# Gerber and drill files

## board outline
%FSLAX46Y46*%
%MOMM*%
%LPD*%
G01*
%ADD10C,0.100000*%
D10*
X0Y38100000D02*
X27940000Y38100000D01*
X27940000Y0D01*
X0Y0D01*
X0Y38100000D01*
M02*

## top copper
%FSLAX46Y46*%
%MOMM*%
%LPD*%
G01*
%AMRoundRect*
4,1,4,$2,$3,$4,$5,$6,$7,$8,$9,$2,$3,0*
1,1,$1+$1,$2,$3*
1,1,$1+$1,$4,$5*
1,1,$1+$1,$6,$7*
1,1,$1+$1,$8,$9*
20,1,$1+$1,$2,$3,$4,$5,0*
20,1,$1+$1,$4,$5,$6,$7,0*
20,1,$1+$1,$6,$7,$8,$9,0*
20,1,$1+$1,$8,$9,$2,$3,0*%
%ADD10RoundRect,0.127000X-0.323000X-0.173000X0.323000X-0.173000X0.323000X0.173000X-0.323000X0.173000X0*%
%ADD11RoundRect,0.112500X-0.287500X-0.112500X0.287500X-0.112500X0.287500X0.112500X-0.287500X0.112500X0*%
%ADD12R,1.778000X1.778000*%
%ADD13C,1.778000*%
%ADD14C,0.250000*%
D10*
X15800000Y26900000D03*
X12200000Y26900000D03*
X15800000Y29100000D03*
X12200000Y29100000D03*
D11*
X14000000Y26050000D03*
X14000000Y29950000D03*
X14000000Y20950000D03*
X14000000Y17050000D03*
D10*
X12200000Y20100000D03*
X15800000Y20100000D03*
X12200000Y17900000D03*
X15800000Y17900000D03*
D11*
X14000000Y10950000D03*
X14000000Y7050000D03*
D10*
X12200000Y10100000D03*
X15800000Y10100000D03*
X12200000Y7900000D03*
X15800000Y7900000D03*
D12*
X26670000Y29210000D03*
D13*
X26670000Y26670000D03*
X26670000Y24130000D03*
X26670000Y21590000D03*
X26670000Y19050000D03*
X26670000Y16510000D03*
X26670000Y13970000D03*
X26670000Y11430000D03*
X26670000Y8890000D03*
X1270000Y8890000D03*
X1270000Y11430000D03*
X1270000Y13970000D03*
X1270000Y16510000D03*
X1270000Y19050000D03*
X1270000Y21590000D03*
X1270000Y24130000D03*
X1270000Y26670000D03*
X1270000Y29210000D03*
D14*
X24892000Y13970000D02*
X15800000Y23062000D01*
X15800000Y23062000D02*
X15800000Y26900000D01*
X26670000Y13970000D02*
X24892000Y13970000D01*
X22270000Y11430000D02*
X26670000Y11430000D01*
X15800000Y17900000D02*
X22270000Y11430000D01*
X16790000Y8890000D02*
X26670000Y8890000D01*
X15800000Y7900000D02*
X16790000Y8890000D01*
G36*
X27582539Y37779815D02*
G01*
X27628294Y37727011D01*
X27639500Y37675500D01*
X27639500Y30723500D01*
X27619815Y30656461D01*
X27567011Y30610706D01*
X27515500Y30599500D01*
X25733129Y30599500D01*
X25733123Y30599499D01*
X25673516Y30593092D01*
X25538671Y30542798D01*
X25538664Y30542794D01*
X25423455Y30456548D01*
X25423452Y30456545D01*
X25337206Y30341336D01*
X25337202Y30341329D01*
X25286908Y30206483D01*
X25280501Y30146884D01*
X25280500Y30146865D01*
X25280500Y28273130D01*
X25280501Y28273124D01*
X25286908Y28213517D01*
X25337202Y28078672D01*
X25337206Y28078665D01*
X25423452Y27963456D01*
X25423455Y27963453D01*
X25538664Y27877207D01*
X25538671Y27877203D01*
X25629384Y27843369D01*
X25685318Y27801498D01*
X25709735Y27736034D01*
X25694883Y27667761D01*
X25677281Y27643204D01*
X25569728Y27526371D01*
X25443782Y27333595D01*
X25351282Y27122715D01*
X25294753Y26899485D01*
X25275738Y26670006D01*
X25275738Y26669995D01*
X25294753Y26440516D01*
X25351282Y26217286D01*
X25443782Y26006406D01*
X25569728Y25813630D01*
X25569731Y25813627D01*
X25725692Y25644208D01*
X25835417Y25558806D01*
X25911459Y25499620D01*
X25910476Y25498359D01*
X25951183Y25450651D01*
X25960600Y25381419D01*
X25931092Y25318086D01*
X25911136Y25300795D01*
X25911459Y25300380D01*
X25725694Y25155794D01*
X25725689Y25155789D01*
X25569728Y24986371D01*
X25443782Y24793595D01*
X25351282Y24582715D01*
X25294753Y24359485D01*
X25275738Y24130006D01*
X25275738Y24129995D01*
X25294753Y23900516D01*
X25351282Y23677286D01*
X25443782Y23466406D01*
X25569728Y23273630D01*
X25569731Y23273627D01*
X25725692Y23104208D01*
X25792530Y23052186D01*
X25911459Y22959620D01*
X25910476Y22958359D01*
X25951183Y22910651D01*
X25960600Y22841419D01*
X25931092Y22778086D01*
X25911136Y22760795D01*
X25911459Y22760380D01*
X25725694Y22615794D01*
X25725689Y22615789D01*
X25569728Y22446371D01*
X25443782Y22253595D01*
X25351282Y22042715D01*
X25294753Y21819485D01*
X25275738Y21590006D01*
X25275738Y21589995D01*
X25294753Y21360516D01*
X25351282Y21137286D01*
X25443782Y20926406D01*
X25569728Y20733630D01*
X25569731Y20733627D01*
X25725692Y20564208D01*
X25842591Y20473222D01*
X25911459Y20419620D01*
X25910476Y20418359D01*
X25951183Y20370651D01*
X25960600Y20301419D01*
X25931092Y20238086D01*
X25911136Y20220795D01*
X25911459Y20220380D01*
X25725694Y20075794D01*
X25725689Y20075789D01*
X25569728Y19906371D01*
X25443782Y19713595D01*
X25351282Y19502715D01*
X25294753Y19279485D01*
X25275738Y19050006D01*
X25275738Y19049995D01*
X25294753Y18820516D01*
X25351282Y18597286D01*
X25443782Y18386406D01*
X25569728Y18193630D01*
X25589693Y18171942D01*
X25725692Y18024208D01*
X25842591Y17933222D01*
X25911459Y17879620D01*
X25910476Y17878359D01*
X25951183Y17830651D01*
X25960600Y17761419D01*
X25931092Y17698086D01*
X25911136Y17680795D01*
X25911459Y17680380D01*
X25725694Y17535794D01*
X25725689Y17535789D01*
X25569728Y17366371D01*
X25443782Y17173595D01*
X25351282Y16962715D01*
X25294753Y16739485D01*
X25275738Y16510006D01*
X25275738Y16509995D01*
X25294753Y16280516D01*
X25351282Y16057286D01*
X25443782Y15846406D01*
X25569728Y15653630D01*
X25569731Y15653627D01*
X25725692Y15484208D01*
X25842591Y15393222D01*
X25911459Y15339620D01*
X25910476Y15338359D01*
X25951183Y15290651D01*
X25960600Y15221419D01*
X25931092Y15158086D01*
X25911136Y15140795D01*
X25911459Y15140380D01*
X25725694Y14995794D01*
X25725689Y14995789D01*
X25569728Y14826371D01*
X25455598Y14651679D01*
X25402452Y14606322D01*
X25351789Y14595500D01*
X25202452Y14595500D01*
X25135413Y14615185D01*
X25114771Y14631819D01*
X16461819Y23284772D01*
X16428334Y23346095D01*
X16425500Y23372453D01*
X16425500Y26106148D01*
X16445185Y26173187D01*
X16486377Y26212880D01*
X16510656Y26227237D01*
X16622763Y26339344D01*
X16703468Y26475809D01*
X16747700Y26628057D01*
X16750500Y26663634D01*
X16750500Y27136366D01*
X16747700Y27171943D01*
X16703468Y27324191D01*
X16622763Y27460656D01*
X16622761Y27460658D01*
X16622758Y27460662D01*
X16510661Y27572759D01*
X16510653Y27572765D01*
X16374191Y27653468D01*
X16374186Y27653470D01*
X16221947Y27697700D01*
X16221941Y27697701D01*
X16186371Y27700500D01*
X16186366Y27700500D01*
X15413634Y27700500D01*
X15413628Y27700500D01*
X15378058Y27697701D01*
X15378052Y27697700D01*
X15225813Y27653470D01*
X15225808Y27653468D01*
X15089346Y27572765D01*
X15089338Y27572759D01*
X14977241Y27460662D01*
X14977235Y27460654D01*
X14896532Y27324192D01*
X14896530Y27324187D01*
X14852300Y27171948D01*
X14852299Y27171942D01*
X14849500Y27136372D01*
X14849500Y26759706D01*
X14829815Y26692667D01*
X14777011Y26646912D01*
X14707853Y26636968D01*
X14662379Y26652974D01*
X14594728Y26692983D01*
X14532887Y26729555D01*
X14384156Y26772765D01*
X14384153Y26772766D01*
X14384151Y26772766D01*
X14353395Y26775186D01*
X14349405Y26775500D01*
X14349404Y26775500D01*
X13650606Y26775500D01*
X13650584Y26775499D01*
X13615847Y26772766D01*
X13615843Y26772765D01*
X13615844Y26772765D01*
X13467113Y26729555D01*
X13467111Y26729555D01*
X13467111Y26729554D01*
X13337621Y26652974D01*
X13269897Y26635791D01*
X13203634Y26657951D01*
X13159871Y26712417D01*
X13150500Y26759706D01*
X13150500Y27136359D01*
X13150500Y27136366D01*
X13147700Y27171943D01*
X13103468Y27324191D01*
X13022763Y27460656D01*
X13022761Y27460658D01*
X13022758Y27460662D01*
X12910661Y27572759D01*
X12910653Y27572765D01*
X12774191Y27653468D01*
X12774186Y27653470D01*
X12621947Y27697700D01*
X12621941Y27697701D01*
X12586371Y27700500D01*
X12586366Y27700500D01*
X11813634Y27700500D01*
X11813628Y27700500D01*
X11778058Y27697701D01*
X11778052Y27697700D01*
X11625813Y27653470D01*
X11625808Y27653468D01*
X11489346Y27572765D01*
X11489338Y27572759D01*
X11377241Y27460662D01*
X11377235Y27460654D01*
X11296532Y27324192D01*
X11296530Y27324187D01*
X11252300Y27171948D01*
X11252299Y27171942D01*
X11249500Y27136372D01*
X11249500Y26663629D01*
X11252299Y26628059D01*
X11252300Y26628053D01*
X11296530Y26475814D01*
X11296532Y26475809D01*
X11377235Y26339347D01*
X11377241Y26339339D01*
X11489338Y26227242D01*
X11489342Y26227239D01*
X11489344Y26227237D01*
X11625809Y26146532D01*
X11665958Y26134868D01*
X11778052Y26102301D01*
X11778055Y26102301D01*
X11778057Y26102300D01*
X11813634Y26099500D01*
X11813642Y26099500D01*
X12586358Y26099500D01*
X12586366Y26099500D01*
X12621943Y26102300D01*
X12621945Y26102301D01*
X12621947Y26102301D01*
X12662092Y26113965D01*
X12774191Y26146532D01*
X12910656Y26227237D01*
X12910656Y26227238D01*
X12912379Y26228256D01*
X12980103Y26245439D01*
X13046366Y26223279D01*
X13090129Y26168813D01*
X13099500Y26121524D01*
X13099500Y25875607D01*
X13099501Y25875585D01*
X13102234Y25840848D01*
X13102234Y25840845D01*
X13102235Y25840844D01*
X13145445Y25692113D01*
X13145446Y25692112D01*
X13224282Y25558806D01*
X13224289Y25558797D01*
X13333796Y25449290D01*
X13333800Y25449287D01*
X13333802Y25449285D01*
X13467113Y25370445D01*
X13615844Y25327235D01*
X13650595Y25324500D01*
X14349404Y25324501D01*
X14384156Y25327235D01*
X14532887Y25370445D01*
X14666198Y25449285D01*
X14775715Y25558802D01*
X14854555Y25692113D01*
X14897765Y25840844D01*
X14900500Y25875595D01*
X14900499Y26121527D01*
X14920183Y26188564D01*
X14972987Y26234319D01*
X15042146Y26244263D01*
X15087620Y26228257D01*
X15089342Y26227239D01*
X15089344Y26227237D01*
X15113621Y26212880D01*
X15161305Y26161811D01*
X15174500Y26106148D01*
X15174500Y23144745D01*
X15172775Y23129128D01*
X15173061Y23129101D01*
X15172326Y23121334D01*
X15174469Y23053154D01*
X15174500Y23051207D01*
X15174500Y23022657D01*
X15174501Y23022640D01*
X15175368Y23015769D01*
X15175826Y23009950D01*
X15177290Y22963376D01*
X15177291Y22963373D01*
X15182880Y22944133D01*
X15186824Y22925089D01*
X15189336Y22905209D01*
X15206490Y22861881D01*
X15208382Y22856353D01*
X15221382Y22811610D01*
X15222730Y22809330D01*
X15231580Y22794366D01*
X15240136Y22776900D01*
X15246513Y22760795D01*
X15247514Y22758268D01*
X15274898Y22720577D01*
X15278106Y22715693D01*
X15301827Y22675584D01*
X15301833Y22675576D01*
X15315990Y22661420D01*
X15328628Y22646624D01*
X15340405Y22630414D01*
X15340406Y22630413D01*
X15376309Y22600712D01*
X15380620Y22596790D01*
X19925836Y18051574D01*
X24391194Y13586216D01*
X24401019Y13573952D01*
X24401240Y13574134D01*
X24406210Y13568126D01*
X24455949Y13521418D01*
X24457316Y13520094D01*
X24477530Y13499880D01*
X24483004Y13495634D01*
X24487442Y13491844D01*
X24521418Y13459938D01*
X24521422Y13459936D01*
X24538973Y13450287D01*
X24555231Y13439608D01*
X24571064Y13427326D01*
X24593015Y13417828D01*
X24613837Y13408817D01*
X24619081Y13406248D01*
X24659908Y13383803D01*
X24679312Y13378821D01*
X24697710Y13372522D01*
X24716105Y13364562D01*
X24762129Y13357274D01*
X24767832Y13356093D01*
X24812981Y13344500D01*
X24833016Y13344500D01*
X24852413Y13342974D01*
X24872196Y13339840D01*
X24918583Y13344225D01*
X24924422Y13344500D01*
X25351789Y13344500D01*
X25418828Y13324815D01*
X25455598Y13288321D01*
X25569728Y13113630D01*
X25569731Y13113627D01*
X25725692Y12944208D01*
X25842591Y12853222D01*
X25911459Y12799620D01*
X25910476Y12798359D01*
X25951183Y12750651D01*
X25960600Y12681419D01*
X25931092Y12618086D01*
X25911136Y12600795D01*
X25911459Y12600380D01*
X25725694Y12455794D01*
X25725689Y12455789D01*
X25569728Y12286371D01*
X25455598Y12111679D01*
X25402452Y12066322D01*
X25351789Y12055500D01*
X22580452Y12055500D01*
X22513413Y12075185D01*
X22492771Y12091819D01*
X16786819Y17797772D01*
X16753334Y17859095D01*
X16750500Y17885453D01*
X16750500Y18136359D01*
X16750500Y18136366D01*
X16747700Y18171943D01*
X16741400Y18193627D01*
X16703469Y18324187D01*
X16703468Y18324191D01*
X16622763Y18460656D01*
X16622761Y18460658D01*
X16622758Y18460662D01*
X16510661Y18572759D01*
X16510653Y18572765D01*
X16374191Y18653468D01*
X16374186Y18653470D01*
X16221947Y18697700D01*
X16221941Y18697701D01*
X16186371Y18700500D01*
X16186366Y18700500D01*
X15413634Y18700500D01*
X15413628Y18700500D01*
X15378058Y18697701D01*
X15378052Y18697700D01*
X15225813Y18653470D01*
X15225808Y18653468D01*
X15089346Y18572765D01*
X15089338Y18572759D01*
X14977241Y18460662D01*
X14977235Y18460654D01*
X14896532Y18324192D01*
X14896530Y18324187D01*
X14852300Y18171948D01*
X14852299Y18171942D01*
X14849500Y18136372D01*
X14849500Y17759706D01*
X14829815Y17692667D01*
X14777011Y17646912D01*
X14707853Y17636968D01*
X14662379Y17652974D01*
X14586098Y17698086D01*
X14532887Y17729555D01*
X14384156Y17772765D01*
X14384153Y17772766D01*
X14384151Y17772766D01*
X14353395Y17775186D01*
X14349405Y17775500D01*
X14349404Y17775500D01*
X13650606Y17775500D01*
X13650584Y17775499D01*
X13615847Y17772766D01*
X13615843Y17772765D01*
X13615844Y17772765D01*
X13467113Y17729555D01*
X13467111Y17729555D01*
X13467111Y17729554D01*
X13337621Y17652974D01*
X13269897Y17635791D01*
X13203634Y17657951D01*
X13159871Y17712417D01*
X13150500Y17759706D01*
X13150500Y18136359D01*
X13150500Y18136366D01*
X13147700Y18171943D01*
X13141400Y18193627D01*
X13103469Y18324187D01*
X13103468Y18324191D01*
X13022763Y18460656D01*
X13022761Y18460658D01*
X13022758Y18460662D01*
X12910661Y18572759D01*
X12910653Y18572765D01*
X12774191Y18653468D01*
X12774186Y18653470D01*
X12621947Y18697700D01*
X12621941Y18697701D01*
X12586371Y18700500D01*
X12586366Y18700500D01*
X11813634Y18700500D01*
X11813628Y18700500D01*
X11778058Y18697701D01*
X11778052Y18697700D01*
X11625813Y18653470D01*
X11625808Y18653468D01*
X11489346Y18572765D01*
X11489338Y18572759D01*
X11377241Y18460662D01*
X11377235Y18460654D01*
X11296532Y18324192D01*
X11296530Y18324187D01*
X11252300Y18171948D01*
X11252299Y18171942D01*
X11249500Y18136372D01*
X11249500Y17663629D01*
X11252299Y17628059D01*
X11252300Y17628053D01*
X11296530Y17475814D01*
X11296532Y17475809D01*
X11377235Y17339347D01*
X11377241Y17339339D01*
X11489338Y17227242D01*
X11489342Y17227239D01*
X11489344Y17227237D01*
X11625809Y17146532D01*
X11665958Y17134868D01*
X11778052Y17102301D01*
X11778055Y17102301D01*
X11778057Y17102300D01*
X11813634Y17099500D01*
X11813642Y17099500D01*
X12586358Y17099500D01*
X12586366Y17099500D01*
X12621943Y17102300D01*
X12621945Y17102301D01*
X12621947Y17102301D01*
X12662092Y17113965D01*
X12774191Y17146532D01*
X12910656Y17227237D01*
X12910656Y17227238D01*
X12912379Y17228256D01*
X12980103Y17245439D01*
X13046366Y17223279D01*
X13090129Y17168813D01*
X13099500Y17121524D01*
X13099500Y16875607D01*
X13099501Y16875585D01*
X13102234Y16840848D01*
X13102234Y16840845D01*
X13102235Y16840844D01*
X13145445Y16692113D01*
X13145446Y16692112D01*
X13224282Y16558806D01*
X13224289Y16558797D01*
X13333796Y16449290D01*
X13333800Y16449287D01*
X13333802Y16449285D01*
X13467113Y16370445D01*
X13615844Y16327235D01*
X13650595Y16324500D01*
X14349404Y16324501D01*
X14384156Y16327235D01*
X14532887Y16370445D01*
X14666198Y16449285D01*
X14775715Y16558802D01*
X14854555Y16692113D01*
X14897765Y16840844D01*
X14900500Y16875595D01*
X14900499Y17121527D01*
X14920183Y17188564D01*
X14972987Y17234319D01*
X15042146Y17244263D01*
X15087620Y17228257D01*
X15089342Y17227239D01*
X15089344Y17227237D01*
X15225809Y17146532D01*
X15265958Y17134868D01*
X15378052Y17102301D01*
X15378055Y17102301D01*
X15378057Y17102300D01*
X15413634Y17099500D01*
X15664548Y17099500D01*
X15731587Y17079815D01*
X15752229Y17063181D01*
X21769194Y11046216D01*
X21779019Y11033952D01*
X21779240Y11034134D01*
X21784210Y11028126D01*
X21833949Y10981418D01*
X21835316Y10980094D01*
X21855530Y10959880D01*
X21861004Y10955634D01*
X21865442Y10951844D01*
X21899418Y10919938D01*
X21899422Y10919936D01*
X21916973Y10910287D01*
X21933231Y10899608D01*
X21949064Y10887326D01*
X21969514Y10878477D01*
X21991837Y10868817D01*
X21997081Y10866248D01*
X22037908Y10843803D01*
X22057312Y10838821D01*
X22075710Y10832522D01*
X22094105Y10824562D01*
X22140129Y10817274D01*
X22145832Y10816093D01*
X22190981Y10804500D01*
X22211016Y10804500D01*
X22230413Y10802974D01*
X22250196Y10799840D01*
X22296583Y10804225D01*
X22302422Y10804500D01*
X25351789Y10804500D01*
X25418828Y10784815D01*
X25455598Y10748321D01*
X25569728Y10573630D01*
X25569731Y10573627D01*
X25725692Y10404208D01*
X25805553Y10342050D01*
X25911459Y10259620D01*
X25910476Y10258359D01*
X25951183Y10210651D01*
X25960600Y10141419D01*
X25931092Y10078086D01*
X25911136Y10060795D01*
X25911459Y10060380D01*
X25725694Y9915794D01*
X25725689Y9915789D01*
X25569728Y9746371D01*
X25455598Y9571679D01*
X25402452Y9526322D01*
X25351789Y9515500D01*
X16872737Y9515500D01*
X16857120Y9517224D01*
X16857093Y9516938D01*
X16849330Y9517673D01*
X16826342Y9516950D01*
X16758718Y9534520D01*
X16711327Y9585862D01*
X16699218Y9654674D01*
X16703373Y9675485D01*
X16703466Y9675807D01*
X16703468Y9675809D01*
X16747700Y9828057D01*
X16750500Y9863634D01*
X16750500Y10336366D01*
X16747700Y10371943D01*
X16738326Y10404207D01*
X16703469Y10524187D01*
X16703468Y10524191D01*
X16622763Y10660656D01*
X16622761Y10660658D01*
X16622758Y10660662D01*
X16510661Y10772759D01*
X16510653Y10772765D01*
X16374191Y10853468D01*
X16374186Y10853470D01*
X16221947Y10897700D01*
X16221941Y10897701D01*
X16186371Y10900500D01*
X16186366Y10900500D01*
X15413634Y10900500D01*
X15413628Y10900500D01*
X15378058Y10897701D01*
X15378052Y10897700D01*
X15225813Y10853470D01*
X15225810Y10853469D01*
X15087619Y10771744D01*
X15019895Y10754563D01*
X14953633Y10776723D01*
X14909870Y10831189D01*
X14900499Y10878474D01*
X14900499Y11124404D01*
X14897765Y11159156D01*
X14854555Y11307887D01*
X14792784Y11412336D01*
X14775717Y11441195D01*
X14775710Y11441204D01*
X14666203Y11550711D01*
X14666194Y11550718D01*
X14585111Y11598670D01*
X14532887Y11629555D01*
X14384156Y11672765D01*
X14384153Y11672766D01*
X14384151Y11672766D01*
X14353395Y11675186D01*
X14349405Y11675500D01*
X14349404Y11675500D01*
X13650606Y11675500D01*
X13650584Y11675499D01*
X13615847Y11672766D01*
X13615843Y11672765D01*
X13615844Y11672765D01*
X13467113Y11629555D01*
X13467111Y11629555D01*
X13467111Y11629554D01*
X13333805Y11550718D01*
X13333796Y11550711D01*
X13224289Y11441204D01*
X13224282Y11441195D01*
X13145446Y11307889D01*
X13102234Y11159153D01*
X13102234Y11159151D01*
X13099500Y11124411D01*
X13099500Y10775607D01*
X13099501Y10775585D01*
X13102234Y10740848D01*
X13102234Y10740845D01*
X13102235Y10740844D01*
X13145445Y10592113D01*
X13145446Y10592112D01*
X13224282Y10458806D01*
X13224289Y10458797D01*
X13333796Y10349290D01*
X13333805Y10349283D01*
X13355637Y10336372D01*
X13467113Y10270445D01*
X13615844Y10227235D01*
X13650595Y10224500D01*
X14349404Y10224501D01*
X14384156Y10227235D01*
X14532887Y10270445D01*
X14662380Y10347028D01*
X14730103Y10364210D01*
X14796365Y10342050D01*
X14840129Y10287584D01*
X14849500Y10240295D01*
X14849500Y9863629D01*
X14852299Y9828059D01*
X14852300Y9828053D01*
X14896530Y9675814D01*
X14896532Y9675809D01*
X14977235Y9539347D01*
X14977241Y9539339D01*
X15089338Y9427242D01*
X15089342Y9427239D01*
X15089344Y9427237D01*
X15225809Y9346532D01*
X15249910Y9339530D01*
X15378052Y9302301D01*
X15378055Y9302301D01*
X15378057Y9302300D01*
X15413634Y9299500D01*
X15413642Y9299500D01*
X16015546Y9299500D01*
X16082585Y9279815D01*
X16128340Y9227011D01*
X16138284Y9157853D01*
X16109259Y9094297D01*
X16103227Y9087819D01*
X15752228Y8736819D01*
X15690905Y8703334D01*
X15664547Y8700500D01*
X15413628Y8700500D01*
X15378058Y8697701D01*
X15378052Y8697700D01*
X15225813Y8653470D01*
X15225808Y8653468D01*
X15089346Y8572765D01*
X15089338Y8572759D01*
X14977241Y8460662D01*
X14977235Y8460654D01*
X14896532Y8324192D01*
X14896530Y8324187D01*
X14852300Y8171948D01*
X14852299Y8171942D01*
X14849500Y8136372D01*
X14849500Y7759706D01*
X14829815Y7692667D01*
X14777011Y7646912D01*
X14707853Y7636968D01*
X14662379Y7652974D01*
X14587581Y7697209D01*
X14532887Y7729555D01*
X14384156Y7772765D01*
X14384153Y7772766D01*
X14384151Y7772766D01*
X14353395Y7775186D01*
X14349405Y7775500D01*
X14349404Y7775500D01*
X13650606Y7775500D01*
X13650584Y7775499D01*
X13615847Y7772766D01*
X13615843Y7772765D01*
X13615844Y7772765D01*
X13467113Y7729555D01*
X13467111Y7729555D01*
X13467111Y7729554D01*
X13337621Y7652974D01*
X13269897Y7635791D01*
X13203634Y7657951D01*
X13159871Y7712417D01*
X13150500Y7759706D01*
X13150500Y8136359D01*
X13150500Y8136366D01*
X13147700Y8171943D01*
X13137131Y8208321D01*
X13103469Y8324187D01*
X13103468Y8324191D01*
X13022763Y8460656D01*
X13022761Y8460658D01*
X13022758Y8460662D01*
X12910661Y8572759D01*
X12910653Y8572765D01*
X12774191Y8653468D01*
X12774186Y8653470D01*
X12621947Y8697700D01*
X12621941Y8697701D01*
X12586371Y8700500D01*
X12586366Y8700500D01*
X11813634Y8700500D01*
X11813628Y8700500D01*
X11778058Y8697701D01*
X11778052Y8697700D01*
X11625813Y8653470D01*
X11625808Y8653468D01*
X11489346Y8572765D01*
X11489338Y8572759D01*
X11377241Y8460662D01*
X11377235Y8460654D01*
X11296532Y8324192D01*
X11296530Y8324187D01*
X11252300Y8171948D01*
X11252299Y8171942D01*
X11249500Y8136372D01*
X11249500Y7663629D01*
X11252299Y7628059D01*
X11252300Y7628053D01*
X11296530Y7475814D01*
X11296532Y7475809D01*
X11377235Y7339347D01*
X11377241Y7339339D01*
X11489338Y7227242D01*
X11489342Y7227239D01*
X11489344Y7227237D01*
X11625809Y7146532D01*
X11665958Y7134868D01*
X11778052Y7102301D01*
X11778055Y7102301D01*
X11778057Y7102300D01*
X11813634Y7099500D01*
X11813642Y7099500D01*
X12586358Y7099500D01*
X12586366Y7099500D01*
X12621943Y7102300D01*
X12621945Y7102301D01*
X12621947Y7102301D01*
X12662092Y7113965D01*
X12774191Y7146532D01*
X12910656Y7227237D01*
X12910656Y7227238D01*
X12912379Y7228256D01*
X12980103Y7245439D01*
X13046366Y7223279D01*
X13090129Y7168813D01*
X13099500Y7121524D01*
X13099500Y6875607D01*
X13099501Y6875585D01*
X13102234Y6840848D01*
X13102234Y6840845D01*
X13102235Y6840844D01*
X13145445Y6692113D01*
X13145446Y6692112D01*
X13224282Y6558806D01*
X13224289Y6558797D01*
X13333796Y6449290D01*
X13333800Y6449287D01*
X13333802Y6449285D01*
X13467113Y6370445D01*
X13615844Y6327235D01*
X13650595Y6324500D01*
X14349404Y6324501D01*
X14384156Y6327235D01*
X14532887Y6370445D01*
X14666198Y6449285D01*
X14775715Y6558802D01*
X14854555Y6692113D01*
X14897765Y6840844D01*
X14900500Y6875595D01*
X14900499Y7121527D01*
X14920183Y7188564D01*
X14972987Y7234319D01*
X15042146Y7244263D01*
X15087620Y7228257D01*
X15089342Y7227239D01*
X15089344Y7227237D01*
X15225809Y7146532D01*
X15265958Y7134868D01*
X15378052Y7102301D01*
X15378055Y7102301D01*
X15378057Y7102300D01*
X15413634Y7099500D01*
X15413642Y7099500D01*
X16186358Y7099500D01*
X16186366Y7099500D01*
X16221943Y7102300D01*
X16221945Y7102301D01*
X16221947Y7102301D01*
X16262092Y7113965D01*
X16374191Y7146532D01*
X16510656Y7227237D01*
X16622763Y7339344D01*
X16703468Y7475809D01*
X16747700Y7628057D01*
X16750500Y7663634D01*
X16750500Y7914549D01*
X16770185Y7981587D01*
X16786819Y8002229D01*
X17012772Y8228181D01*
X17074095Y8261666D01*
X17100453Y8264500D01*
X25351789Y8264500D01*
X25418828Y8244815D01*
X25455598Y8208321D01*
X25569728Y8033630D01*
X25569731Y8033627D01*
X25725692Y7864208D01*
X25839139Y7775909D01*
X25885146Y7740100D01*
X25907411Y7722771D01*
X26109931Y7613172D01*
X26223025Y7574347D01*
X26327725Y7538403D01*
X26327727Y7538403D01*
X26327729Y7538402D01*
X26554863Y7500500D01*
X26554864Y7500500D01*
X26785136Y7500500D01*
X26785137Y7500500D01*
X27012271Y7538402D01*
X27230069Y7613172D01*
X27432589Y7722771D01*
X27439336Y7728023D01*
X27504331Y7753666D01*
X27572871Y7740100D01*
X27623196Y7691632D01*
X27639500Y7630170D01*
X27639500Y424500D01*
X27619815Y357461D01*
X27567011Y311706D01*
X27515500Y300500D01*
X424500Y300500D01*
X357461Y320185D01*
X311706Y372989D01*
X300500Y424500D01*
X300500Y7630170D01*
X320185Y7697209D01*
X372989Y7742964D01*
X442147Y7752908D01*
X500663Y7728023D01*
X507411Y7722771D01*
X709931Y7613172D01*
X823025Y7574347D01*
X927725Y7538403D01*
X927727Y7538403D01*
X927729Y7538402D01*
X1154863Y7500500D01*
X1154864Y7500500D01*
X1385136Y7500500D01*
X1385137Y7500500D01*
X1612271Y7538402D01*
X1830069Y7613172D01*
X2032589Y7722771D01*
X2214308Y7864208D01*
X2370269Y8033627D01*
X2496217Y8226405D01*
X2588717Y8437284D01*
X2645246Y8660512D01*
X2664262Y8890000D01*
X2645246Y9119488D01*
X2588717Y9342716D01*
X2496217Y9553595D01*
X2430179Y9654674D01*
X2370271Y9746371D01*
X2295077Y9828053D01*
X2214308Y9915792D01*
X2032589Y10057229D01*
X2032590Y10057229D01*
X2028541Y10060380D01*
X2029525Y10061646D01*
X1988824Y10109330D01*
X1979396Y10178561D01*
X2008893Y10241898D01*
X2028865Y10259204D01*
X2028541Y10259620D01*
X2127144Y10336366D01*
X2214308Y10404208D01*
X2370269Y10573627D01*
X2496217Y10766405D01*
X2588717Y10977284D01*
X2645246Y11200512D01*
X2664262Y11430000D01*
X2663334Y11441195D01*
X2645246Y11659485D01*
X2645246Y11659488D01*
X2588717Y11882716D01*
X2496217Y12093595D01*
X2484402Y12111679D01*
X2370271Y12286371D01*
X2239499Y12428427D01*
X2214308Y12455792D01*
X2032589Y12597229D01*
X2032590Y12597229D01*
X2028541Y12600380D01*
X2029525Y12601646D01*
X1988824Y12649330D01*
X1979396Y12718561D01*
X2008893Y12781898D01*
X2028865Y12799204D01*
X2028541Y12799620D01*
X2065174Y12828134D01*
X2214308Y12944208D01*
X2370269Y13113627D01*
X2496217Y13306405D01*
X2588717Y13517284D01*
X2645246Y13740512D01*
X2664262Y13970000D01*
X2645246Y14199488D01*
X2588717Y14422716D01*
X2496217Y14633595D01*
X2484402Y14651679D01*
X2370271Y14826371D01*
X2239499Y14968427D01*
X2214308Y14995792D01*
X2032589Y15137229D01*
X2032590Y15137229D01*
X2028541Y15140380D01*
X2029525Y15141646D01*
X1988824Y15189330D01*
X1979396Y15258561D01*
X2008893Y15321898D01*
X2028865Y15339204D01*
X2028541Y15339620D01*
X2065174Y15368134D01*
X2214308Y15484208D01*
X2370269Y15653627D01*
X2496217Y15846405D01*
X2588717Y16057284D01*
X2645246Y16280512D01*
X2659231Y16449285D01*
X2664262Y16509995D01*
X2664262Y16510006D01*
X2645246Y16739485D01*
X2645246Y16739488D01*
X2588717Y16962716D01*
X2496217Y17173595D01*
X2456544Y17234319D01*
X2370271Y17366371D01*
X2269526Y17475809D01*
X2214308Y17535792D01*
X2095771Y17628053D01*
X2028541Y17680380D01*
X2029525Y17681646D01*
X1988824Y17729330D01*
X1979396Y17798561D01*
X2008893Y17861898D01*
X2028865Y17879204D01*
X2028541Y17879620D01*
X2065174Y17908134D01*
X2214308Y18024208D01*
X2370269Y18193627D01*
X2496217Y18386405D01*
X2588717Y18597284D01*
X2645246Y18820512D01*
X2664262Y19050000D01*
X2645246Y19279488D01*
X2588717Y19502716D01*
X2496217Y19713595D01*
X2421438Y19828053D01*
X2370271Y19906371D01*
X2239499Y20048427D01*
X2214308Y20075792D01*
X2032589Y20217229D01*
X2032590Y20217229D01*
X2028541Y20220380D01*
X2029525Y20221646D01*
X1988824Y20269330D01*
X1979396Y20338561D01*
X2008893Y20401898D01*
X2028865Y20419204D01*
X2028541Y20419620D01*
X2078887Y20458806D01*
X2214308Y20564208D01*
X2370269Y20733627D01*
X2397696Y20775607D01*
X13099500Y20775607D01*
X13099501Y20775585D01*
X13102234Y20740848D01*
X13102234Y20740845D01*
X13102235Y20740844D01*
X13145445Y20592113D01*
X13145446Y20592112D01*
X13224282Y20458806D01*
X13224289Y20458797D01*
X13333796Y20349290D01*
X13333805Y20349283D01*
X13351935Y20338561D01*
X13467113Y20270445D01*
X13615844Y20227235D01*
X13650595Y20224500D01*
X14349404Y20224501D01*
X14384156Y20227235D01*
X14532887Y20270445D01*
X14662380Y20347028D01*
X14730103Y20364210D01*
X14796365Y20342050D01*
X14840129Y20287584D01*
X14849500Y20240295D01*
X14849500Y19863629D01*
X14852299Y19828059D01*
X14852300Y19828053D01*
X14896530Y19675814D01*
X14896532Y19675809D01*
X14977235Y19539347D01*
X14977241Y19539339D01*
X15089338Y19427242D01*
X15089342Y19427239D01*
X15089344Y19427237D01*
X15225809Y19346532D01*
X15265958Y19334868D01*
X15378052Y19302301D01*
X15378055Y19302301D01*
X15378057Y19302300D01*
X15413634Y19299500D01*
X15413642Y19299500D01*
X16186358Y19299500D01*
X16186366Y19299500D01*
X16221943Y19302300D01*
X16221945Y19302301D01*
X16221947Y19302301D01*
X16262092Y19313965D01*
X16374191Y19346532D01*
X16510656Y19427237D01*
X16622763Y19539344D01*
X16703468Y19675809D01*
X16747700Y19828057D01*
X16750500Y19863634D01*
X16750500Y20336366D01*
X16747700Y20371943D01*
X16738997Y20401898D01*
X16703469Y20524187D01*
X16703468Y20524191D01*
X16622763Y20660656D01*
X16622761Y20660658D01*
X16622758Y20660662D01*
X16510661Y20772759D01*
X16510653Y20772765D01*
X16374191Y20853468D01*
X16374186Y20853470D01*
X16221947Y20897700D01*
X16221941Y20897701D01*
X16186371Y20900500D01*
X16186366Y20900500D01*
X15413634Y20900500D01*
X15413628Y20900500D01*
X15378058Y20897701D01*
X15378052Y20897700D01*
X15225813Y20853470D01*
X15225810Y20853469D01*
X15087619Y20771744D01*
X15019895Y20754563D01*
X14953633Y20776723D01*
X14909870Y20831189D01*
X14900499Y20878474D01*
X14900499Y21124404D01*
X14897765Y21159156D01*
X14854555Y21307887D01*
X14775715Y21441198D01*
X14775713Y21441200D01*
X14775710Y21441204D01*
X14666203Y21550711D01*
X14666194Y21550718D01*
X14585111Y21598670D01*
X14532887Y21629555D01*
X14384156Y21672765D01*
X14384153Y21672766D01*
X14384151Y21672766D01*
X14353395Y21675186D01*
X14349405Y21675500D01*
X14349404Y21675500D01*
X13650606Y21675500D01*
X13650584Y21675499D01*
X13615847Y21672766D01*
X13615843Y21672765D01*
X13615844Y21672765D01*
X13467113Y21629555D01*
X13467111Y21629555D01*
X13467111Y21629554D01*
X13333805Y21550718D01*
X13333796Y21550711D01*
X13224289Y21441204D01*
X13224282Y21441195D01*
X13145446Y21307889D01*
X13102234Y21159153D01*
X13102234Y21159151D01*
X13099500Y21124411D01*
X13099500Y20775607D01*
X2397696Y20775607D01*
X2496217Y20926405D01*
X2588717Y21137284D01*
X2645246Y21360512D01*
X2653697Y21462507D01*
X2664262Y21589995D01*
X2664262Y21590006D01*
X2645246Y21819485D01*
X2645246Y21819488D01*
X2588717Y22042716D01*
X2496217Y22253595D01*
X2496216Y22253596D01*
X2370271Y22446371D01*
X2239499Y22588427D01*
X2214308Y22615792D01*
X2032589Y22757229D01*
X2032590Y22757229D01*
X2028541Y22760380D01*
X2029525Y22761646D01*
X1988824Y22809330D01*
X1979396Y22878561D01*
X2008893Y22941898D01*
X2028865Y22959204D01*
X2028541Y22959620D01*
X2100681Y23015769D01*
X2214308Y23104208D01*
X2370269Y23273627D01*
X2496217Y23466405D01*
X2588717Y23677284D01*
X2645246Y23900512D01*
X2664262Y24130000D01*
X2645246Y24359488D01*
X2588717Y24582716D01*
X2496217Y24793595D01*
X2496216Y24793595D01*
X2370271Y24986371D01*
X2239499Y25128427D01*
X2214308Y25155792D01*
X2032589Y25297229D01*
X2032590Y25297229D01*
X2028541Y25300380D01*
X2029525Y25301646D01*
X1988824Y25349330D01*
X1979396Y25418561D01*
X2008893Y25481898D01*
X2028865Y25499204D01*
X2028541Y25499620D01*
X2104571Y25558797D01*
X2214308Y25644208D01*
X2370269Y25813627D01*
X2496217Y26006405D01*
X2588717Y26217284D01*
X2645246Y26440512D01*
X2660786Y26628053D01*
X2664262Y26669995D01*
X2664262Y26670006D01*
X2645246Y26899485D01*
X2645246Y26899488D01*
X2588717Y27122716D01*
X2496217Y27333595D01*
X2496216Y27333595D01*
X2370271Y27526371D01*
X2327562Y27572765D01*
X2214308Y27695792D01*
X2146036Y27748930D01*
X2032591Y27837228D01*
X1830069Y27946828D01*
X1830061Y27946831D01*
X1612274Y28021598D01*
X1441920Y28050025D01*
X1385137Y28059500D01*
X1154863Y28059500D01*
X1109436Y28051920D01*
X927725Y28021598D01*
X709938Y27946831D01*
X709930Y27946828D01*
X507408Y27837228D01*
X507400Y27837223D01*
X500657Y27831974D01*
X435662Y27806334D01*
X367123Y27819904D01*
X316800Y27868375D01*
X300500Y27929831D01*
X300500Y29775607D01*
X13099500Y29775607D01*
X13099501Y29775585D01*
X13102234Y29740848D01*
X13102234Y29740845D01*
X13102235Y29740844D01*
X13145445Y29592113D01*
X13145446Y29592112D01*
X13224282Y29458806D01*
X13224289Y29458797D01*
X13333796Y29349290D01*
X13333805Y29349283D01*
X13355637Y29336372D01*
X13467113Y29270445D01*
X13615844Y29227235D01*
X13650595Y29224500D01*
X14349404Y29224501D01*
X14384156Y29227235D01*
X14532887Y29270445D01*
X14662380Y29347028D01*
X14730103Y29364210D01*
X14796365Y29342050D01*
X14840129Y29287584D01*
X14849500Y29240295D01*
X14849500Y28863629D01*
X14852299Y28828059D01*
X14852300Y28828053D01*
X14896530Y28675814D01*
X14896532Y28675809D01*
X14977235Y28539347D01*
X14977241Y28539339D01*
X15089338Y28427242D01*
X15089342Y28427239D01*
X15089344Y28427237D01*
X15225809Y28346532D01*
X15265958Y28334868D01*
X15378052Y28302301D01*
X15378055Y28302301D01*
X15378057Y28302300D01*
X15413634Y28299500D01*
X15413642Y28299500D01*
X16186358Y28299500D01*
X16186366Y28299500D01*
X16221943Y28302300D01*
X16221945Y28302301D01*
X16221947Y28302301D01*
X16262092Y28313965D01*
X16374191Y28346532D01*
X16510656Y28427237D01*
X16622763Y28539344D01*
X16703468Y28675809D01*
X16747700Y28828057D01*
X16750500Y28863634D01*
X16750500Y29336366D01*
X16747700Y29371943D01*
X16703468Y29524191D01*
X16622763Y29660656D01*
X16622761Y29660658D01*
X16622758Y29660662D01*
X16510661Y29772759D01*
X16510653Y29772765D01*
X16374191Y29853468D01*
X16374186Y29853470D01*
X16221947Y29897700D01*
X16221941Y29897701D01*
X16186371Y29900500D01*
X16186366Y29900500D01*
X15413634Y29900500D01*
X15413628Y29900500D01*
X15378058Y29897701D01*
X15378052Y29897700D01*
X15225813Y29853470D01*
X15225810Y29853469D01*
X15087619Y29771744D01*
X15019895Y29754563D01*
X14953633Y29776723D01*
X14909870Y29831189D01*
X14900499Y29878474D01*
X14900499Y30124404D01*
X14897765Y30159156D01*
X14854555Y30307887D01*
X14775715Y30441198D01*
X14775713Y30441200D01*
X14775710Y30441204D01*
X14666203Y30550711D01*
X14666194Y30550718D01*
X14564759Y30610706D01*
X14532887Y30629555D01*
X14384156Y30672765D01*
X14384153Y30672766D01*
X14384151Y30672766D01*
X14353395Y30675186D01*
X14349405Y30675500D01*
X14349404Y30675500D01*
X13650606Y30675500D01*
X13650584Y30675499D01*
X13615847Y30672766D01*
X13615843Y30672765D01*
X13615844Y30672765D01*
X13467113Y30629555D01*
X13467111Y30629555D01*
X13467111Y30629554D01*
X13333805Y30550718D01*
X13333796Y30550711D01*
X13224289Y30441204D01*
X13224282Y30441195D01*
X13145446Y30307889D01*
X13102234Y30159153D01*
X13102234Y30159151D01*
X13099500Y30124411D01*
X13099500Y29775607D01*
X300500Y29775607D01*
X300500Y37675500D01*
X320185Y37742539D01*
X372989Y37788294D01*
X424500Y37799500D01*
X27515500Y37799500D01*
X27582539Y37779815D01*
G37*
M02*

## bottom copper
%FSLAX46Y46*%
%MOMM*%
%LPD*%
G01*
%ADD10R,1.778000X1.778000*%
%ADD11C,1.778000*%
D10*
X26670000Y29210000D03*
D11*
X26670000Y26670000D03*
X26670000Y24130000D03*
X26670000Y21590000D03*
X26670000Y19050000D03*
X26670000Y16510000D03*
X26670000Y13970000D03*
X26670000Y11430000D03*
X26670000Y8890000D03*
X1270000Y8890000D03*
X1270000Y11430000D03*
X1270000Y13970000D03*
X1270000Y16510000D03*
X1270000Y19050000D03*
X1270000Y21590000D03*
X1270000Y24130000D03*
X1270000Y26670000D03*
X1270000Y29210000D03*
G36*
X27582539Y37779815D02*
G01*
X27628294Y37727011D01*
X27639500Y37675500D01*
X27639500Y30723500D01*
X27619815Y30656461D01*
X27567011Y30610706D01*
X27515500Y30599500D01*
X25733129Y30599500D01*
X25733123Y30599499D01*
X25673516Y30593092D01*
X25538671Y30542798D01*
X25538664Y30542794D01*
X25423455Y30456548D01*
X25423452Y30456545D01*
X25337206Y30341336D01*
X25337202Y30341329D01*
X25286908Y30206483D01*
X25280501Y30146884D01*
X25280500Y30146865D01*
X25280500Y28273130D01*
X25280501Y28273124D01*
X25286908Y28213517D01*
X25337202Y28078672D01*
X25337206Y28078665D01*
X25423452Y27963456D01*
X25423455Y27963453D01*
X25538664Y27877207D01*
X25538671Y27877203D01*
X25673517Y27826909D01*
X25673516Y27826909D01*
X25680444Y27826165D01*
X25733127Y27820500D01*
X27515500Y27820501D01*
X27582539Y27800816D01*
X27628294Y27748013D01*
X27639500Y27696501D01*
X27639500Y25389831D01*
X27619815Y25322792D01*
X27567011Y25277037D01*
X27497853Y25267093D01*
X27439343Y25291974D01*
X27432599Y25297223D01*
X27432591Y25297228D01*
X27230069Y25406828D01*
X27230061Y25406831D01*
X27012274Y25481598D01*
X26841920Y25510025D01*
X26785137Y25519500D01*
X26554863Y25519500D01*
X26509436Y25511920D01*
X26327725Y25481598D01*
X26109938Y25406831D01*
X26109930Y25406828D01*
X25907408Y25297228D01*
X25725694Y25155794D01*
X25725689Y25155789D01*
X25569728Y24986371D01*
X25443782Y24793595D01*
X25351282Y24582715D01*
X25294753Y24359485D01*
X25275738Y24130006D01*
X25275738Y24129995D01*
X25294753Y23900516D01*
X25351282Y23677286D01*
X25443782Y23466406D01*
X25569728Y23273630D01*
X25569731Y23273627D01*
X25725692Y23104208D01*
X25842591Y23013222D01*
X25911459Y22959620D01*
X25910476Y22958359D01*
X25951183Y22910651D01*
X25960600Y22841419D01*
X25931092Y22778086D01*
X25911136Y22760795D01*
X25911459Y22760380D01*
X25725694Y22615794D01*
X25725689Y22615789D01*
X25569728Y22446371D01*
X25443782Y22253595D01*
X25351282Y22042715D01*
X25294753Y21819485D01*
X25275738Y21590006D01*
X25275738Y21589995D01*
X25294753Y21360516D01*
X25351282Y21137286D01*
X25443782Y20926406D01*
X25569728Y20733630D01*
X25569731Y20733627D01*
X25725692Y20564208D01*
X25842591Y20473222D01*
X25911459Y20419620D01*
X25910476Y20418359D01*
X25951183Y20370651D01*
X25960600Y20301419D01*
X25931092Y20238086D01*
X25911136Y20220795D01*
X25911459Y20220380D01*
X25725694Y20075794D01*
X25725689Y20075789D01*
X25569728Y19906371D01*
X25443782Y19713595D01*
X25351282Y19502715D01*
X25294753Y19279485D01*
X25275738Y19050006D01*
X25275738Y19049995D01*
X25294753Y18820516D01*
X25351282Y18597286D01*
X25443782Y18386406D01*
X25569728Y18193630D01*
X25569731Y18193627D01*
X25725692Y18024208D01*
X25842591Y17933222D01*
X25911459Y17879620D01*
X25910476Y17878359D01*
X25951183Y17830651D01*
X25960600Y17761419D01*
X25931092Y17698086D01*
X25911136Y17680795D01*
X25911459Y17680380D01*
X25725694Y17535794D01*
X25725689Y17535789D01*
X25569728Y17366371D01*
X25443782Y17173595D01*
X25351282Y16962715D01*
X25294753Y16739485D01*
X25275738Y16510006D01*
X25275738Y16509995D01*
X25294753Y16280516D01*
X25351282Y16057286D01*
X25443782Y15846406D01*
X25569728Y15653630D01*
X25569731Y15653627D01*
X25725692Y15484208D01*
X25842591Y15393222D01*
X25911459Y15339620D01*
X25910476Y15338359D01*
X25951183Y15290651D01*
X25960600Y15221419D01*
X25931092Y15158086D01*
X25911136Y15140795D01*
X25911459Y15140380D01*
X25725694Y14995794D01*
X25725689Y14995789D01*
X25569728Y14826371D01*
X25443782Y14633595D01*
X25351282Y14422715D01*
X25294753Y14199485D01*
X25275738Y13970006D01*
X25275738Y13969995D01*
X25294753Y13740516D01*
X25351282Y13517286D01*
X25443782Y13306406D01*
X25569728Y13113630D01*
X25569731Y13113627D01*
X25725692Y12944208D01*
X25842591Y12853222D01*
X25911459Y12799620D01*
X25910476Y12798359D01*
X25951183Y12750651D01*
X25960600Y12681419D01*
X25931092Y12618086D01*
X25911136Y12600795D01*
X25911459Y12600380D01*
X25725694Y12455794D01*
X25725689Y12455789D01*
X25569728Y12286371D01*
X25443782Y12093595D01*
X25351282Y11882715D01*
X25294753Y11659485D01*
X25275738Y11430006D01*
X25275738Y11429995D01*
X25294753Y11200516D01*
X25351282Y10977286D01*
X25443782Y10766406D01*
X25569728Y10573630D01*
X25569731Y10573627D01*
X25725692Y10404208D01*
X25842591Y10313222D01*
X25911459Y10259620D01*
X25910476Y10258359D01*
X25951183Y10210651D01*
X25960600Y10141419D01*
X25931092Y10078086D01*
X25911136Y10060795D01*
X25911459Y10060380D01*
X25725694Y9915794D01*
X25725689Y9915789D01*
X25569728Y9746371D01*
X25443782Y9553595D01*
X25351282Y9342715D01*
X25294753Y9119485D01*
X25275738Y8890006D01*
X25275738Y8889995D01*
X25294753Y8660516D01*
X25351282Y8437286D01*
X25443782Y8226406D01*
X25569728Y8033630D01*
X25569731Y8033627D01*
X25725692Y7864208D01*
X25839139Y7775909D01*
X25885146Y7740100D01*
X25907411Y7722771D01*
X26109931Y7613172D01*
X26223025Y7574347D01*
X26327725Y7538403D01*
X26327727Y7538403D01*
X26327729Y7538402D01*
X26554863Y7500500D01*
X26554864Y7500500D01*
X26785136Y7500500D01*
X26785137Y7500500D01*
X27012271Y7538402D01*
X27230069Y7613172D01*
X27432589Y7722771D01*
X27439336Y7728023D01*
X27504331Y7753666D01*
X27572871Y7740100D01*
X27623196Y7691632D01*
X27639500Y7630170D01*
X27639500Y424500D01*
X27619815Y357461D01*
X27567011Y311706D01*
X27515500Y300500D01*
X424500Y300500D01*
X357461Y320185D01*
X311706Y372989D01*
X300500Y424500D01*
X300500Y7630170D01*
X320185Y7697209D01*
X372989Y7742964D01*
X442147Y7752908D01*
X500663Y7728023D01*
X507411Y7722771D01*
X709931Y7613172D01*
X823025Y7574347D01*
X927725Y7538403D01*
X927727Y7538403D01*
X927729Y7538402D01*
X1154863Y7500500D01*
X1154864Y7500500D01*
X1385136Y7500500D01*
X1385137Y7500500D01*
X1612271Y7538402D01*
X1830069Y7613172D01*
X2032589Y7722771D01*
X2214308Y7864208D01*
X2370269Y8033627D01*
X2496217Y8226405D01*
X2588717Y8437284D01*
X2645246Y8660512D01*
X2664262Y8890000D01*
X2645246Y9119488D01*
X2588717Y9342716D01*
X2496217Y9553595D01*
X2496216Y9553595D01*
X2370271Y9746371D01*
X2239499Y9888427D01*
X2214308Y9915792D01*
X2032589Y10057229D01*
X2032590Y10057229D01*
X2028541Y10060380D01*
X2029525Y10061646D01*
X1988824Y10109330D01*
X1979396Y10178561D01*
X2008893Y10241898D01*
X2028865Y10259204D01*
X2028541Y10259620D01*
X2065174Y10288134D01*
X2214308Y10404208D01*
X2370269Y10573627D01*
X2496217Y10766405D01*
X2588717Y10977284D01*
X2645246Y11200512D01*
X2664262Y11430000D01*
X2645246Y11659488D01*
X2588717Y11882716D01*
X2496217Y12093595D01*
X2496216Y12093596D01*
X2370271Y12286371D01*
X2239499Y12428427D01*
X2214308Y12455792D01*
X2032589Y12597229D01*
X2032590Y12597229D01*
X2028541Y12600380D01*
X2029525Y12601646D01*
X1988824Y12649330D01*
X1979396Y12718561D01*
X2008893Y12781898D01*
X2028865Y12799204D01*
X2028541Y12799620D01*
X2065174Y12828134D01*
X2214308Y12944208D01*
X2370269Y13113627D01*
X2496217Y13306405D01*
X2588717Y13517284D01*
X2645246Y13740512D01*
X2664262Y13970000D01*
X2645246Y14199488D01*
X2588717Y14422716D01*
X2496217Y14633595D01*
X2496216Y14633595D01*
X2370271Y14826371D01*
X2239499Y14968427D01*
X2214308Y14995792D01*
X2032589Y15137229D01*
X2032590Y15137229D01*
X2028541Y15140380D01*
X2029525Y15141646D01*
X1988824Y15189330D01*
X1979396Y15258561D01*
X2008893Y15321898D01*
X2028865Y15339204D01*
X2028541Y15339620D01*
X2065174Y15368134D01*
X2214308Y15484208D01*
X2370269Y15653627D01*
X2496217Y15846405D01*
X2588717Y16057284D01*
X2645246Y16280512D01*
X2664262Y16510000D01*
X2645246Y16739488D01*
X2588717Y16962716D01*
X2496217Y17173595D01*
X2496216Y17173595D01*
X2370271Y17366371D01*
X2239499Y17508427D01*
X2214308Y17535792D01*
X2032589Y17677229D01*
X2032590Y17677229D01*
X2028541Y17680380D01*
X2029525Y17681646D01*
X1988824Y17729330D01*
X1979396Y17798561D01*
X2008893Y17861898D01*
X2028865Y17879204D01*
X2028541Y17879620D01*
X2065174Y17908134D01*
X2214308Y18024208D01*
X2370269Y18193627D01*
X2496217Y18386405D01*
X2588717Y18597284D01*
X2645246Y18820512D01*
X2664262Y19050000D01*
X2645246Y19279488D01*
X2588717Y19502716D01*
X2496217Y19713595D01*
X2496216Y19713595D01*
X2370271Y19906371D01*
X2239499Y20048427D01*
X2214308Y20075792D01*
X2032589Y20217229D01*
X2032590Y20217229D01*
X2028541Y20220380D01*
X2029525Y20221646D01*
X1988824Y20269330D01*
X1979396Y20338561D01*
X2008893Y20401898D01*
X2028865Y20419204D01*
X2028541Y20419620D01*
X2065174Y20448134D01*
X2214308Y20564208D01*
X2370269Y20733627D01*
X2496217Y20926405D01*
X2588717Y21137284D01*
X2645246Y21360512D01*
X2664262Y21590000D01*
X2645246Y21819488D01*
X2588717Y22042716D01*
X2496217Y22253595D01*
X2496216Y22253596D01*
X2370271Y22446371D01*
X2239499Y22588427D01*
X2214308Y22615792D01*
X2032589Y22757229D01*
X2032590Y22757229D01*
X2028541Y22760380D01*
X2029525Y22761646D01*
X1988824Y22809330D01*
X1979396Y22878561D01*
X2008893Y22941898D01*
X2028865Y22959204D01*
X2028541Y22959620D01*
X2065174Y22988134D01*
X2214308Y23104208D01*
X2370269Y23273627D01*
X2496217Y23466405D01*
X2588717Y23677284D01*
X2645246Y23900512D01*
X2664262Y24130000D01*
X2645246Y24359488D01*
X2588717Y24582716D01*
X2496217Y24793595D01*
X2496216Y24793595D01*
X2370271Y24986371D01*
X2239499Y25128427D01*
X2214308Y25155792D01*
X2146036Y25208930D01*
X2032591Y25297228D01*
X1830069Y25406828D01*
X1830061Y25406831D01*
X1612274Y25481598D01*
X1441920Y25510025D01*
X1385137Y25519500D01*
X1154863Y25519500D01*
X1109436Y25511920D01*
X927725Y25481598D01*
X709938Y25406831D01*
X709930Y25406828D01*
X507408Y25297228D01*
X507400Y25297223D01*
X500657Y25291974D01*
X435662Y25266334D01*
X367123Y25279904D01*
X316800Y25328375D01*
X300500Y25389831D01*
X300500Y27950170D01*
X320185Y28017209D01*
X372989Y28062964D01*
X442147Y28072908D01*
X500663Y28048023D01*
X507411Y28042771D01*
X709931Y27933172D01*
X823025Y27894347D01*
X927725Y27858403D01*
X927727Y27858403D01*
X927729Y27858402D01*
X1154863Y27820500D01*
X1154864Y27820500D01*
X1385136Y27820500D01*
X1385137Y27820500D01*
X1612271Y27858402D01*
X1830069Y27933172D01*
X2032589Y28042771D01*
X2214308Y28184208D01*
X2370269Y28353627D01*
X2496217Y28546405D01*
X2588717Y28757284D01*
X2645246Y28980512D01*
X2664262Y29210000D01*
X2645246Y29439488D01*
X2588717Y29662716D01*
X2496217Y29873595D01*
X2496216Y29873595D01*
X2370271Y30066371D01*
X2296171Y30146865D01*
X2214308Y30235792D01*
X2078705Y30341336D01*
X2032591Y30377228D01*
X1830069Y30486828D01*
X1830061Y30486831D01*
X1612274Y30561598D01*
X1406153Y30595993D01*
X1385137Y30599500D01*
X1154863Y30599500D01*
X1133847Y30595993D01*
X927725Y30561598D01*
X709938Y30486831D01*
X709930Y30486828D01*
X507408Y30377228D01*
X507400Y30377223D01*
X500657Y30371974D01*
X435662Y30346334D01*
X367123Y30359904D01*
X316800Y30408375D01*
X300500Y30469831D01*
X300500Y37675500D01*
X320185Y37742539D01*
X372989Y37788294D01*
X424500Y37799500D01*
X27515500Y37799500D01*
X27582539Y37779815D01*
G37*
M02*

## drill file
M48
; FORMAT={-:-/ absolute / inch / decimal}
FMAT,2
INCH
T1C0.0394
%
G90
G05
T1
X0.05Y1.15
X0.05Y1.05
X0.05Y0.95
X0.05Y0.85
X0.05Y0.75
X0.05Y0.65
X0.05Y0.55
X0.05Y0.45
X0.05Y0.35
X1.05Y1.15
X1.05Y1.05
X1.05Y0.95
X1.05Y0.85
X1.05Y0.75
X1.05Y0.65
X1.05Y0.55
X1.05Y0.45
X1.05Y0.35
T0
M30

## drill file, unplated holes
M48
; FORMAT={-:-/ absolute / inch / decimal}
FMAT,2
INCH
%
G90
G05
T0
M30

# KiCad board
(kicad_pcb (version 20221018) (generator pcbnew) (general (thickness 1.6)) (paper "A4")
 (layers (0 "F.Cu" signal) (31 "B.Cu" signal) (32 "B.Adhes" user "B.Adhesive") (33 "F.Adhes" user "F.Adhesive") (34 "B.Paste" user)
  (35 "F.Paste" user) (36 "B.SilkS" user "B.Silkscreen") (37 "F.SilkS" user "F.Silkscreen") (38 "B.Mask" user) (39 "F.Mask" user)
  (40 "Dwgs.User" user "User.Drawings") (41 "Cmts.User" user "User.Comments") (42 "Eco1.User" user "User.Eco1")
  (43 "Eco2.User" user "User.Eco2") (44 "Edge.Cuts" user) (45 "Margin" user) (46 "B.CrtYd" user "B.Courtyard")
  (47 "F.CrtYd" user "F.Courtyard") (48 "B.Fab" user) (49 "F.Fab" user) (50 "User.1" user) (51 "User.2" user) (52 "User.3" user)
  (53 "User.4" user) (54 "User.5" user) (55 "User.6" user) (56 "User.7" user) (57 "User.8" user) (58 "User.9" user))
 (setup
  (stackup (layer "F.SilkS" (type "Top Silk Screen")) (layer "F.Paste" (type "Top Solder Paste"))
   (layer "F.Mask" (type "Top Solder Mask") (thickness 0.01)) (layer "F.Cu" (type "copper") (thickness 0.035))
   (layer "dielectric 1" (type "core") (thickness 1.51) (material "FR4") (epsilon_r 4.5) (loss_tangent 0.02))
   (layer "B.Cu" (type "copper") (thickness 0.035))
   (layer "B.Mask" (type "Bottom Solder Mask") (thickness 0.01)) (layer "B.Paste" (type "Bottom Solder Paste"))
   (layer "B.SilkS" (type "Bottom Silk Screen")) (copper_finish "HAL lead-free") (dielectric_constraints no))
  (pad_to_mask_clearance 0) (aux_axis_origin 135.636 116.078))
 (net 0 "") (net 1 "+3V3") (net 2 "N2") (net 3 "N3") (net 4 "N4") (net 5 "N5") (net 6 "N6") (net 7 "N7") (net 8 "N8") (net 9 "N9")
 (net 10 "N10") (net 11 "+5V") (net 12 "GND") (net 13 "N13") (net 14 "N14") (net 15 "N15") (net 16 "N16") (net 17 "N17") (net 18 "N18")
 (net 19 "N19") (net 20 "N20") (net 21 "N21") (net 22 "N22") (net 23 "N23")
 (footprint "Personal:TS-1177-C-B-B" (layer "F.Cu") (at 149.636 97.078)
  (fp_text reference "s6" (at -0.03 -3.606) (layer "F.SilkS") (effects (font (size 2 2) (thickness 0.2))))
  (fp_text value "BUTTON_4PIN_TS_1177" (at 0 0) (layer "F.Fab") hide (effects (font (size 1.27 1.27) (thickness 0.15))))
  (pad "P$5" smd roundrect (at 0 -1.95) (size 0.8 0.45) (layers "F.Cu" "F.Paste" "F.Mask") (roundrect_rratio 0.25) (thermal_bridge_angle 45))
  (pad "P$6" smd roundrect (at 0 1.95) (size 0.8 0.45) (layers "F.Cu" "F.Paste" "F.Mask") (roundrect_rratio 0.25) (thermal_bridge_angle 45))
  (pad "P1" smd roundrect (at -1.8 -1.1) (size 0.9 0.6) (layers "F.Cu" "F.Paste" "F.Mask") (roundrect_rratio 0.2116666667) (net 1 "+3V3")
   (thermal_bridge_angle 45))
  (pad "P2" smd roundrect (at 1.8 -1.1) (size 0.9 0.6) (layers "F.Cu" "F.Paste" "F.Mask") (roundrect_rratio 0.2116666667) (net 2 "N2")
   (thermal_bridge_angle 45))
  (pad "P3" smd roundrect (at -1.8 1.1) (size 0.9 0.6) (layers "F.Cu" "F.Paste" "F.Mask") (roundrect_rratio 0.2116666667) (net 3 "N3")
   (thermal_bridge_angle 45))
  (pad "P4" smd roundrect (at 1.8 1.1) (size 0.9 0.6) (layers "F.Cu" "F.Paste" "F.Mask") (roundrect_rratio 0.2116666667) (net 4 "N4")
   (thermal_bridge_angle 45)))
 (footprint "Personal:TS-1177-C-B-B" (layer "F.Cu") (at 149.636 88.078)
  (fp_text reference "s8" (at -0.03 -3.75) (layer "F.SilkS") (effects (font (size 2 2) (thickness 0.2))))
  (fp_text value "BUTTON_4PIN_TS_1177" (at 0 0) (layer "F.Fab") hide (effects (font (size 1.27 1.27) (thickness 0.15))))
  (pad "P$5" smd roundrect (at 0 -1.95) (size 0.8 0.45) (layers "F.Cu" "F.Paste" "F.Mask") (roundrect_rratio 0.25) (thermal_bridge_angle 45))
  (pad "P$6" smd roundrect (at 0 1.95) (size 0.8 0.45) (layers "F.Cu" "F.Paste" "F.Mask") (roundrect_rratio 0.25) (thermal_bridge_angle 45))
  (pad "P1" smd roundrect (at -1.8 -1.1) (size 0.9 0.6) (layers "F.Cu" "F.Paste" "F.Mask") (roundrect_rratio 0.2116666667) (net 1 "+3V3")
   (thermal_bridge_angle 45))
  (pad "P2" smd roundrect (at 1.8 -1.1) (size 0.9 0.6) (layers "F.Cu" "F.Paste" "F.Mask") (roundrect_rratio 0.2116666667) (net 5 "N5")
   (thermal_bridge_angle 45))
  (pad "P3" smd roundrect (at -1.8 1.1) (size 0.9 0.6) (layers "F.Cu" "F.Paste" "F.Mask") (roundrect_rratio 0.2116666667) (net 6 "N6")
   (thermal_bridge_angle 45))
  (pad "P4" smd roundrect (at 1.8 1.1) (size 0.9 0.6) (layers "F.Cu" "F.Paste" "F.Mask") (roundrect_rratio 0.2116666667) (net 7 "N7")
   (thermal_bridge_angle 45)))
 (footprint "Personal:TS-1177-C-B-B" (layer "F.Cu") (at 149.636 107.078)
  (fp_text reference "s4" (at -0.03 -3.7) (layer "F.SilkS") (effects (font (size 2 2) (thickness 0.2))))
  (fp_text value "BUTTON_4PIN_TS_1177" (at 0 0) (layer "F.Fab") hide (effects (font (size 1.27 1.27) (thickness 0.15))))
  (pad "P$5" smd roundrect (at 0 -1.95) (size 0.8 0.45) (layers "F.Cu" "F.Paste" "F.Mask") (roundrect_rratio 0.25) (thermal_bridge_angle 45))
  (pad "P$6" smd roundrect (at 0 1.95) (size 0.8 0.45) (layers "F.Cu" "F.Paste" "F.Mask") (roundrect_rratio 0.25) (thermal_bridge_angle 45))
  (pad "P1" smd roundrect (at -1.8 -1.1) (size 0.9 0.6) (layers "F.Cu" "F.Paste" "F.Mask") (roundrect_rratio 0.2116666667) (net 1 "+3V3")
   (thermal_bridge_angle 45))
  (pad "P2" smd roundrect (at 1.8 -1.1) (size 0.9 0.6) (layers "F.Cu" "F.Paste" "F.Mask") (roundrect_rratio 0.2116666667) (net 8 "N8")
   (thermal_bridge_angle 45))
  (pad "P3" smd roundrect (at -1.8 1.1) (size 0.9 0.6) (layers "F.Cu" "F.Paste" "F.Mask") (roundrect_rratio 0.2116666667) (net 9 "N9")
   (thermal_bridge_angle 45))
  (pad "P4" smd roundrect (at 1.8 1.1) (size 0.9 0.6) (layers "F.Cu" "F.Paste" "F.Mask") (roundrect_rratio 0.2116666667) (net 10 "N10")
   (thermal_bridge_angle 45)))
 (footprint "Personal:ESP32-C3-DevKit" (layer "B.Cu") (at 149.606 86.868 180)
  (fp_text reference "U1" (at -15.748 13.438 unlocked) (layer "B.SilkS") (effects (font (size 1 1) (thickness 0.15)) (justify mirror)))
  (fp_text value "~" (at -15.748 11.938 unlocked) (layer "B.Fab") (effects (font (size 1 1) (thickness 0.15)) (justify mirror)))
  (pad "1" thru_hole rect (at -12.7 0 180) (size 1.778 1.778) (drill 1) (layers "*.Cu" "*.Mask") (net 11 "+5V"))
  (pad "2" thru_hole circle (at -12.7 -2.54 180) (size 1.778 1.778) (drill 1) (layers "*.Cu" "*.Mask") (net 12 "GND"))
  (pad "3" thru_hole circle (at -12.7 -5.08 180) (size 1.778 1.778) (drill 1) (layers "*.Cu" "*.Mask") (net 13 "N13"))
  (pad "4" thru_hole circle (at -12.7 -7.62 180) (size 1.778 1.778) (drill 1) (layers "*.Cu" "*.Mask") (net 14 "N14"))
  (pad "5" thru_hole circle (at -12.7 -10.16 180) (size 1.778 1.778) (drill 1) (layers "*.Cu" "*.Mask") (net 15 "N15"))
  (pad "6" thru_hole circle (at -12.7 -12.7 180) (size 1.778 1.778) (drill 1) (layers "*.Cu" "*.Mask") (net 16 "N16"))
  (pad "7" thru_hole circle (at -12.7 -15.24 180) (size 1.778 1.778) (drill 1) (layers "*.Cu" "*.Mask") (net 7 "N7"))
  (pad "8" thru_hole circle (at -12.7 -17.78 180) (size 1.778 1.778) (drill 1) (layers "*.Cu" "*.Mask") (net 4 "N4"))
  (pad "9" thru_hole circle (at -12.7 -20.32 180) (size 1.778 1.778) (drill 1) (layers "*.Cu" "*.Mask") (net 10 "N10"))
  (pad "10" thru_hole circle (at 12.7 -20.32 180) (size 1.778 1.778) (drill 1) (layers "*.Cu" "*.Mask") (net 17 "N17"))
  (pad "11" thru_hole circle (at 12.7 -17.78 180) (size 1.778 1.778) (drill 1) (layers "*.Cu" "*.Mask") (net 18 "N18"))
  (pad "12" thru_hole circle (at 12.7 -15.24 180) (size 1.778 1.778) (drill 1) (layers "*.Cu" "*.Mask") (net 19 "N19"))
  (pad "13" thru_hole circle (at 12.7 -12.7 180) (size 1.778 1.778) (drill 1) (layers "*.Cu" "*.Mask") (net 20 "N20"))
  (pad "14" thru_hole circle (at 12.7 -10.16 180) (size 1.778 1.778) (drill 1) (layers "*.Cu" "*.Mask") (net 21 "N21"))
  (pad "15" thru_hole circle (at 12.7 -7.62 180) (size 1.778 1.778) (drill 1) (layers "*.Cu" "*.Mask") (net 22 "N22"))
  (pad "16" thru_hole circle (at 12.7 -5.08 180) (size 1.778 1.778) (drill 1) (layers "*.Cu" "*.Mask") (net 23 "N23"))
  (pad "17" thru_hole circle (at 12.7 -2.54 180) (size 1.778 1.778) (drill 1) (layers "*.Cu" "*.Mask") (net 12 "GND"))
  (pad "18" thru_hole circle (at 12.7 0 180) (size 1.778 1.778) (drill 1) (layers "*.Cu" "*.Mask") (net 1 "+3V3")))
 (gr_rect (start 135.636 77.978) (end 163.576 116.078) (stroke (width 0.1) (type default)) (fill none) (layer "Edge.Cuts"))
 (segment (start 151.436 108.178) (end 152.426 107.188) (width 0.25) (layer "F.Cu") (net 10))
 (segment (start 152.426 107.188) (end 162.306 107.188) (width 0.25) (layer "F.Cu") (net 10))
 (segment (start 151.436 98.178) (end 157.906 104.648) (width 0.25) (layer "F.Cu") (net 4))
 (segment (start 157.906 104.648) (end 162.306 104.648) (width 0.25) (layer "F.Cu") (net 4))
 (segment (start 151.436 93.016) (end 151.436 89.178) (width 0.25) (layer "F.Cu") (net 7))
 (segment (start 162.306 102.108) (end 160.528 102.108) (width 0.25) (layer "F.Cu") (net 7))
 (segment (start 160.528 102.108) (end 151.436 93.016) (width 0.25) (layer "F.Cu") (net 7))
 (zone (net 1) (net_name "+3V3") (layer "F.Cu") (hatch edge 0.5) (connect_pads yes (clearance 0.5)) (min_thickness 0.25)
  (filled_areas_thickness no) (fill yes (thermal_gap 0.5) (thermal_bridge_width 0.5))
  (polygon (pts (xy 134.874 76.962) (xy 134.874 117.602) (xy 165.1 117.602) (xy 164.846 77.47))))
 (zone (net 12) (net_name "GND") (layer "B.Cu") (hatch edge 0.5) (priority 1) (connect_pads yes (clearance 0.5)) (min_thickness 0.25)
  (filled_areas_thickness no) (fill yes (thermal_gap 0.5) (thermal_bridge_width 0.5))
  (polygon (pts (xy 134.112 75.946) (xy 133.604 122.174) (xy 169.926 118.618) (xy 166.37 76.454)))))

